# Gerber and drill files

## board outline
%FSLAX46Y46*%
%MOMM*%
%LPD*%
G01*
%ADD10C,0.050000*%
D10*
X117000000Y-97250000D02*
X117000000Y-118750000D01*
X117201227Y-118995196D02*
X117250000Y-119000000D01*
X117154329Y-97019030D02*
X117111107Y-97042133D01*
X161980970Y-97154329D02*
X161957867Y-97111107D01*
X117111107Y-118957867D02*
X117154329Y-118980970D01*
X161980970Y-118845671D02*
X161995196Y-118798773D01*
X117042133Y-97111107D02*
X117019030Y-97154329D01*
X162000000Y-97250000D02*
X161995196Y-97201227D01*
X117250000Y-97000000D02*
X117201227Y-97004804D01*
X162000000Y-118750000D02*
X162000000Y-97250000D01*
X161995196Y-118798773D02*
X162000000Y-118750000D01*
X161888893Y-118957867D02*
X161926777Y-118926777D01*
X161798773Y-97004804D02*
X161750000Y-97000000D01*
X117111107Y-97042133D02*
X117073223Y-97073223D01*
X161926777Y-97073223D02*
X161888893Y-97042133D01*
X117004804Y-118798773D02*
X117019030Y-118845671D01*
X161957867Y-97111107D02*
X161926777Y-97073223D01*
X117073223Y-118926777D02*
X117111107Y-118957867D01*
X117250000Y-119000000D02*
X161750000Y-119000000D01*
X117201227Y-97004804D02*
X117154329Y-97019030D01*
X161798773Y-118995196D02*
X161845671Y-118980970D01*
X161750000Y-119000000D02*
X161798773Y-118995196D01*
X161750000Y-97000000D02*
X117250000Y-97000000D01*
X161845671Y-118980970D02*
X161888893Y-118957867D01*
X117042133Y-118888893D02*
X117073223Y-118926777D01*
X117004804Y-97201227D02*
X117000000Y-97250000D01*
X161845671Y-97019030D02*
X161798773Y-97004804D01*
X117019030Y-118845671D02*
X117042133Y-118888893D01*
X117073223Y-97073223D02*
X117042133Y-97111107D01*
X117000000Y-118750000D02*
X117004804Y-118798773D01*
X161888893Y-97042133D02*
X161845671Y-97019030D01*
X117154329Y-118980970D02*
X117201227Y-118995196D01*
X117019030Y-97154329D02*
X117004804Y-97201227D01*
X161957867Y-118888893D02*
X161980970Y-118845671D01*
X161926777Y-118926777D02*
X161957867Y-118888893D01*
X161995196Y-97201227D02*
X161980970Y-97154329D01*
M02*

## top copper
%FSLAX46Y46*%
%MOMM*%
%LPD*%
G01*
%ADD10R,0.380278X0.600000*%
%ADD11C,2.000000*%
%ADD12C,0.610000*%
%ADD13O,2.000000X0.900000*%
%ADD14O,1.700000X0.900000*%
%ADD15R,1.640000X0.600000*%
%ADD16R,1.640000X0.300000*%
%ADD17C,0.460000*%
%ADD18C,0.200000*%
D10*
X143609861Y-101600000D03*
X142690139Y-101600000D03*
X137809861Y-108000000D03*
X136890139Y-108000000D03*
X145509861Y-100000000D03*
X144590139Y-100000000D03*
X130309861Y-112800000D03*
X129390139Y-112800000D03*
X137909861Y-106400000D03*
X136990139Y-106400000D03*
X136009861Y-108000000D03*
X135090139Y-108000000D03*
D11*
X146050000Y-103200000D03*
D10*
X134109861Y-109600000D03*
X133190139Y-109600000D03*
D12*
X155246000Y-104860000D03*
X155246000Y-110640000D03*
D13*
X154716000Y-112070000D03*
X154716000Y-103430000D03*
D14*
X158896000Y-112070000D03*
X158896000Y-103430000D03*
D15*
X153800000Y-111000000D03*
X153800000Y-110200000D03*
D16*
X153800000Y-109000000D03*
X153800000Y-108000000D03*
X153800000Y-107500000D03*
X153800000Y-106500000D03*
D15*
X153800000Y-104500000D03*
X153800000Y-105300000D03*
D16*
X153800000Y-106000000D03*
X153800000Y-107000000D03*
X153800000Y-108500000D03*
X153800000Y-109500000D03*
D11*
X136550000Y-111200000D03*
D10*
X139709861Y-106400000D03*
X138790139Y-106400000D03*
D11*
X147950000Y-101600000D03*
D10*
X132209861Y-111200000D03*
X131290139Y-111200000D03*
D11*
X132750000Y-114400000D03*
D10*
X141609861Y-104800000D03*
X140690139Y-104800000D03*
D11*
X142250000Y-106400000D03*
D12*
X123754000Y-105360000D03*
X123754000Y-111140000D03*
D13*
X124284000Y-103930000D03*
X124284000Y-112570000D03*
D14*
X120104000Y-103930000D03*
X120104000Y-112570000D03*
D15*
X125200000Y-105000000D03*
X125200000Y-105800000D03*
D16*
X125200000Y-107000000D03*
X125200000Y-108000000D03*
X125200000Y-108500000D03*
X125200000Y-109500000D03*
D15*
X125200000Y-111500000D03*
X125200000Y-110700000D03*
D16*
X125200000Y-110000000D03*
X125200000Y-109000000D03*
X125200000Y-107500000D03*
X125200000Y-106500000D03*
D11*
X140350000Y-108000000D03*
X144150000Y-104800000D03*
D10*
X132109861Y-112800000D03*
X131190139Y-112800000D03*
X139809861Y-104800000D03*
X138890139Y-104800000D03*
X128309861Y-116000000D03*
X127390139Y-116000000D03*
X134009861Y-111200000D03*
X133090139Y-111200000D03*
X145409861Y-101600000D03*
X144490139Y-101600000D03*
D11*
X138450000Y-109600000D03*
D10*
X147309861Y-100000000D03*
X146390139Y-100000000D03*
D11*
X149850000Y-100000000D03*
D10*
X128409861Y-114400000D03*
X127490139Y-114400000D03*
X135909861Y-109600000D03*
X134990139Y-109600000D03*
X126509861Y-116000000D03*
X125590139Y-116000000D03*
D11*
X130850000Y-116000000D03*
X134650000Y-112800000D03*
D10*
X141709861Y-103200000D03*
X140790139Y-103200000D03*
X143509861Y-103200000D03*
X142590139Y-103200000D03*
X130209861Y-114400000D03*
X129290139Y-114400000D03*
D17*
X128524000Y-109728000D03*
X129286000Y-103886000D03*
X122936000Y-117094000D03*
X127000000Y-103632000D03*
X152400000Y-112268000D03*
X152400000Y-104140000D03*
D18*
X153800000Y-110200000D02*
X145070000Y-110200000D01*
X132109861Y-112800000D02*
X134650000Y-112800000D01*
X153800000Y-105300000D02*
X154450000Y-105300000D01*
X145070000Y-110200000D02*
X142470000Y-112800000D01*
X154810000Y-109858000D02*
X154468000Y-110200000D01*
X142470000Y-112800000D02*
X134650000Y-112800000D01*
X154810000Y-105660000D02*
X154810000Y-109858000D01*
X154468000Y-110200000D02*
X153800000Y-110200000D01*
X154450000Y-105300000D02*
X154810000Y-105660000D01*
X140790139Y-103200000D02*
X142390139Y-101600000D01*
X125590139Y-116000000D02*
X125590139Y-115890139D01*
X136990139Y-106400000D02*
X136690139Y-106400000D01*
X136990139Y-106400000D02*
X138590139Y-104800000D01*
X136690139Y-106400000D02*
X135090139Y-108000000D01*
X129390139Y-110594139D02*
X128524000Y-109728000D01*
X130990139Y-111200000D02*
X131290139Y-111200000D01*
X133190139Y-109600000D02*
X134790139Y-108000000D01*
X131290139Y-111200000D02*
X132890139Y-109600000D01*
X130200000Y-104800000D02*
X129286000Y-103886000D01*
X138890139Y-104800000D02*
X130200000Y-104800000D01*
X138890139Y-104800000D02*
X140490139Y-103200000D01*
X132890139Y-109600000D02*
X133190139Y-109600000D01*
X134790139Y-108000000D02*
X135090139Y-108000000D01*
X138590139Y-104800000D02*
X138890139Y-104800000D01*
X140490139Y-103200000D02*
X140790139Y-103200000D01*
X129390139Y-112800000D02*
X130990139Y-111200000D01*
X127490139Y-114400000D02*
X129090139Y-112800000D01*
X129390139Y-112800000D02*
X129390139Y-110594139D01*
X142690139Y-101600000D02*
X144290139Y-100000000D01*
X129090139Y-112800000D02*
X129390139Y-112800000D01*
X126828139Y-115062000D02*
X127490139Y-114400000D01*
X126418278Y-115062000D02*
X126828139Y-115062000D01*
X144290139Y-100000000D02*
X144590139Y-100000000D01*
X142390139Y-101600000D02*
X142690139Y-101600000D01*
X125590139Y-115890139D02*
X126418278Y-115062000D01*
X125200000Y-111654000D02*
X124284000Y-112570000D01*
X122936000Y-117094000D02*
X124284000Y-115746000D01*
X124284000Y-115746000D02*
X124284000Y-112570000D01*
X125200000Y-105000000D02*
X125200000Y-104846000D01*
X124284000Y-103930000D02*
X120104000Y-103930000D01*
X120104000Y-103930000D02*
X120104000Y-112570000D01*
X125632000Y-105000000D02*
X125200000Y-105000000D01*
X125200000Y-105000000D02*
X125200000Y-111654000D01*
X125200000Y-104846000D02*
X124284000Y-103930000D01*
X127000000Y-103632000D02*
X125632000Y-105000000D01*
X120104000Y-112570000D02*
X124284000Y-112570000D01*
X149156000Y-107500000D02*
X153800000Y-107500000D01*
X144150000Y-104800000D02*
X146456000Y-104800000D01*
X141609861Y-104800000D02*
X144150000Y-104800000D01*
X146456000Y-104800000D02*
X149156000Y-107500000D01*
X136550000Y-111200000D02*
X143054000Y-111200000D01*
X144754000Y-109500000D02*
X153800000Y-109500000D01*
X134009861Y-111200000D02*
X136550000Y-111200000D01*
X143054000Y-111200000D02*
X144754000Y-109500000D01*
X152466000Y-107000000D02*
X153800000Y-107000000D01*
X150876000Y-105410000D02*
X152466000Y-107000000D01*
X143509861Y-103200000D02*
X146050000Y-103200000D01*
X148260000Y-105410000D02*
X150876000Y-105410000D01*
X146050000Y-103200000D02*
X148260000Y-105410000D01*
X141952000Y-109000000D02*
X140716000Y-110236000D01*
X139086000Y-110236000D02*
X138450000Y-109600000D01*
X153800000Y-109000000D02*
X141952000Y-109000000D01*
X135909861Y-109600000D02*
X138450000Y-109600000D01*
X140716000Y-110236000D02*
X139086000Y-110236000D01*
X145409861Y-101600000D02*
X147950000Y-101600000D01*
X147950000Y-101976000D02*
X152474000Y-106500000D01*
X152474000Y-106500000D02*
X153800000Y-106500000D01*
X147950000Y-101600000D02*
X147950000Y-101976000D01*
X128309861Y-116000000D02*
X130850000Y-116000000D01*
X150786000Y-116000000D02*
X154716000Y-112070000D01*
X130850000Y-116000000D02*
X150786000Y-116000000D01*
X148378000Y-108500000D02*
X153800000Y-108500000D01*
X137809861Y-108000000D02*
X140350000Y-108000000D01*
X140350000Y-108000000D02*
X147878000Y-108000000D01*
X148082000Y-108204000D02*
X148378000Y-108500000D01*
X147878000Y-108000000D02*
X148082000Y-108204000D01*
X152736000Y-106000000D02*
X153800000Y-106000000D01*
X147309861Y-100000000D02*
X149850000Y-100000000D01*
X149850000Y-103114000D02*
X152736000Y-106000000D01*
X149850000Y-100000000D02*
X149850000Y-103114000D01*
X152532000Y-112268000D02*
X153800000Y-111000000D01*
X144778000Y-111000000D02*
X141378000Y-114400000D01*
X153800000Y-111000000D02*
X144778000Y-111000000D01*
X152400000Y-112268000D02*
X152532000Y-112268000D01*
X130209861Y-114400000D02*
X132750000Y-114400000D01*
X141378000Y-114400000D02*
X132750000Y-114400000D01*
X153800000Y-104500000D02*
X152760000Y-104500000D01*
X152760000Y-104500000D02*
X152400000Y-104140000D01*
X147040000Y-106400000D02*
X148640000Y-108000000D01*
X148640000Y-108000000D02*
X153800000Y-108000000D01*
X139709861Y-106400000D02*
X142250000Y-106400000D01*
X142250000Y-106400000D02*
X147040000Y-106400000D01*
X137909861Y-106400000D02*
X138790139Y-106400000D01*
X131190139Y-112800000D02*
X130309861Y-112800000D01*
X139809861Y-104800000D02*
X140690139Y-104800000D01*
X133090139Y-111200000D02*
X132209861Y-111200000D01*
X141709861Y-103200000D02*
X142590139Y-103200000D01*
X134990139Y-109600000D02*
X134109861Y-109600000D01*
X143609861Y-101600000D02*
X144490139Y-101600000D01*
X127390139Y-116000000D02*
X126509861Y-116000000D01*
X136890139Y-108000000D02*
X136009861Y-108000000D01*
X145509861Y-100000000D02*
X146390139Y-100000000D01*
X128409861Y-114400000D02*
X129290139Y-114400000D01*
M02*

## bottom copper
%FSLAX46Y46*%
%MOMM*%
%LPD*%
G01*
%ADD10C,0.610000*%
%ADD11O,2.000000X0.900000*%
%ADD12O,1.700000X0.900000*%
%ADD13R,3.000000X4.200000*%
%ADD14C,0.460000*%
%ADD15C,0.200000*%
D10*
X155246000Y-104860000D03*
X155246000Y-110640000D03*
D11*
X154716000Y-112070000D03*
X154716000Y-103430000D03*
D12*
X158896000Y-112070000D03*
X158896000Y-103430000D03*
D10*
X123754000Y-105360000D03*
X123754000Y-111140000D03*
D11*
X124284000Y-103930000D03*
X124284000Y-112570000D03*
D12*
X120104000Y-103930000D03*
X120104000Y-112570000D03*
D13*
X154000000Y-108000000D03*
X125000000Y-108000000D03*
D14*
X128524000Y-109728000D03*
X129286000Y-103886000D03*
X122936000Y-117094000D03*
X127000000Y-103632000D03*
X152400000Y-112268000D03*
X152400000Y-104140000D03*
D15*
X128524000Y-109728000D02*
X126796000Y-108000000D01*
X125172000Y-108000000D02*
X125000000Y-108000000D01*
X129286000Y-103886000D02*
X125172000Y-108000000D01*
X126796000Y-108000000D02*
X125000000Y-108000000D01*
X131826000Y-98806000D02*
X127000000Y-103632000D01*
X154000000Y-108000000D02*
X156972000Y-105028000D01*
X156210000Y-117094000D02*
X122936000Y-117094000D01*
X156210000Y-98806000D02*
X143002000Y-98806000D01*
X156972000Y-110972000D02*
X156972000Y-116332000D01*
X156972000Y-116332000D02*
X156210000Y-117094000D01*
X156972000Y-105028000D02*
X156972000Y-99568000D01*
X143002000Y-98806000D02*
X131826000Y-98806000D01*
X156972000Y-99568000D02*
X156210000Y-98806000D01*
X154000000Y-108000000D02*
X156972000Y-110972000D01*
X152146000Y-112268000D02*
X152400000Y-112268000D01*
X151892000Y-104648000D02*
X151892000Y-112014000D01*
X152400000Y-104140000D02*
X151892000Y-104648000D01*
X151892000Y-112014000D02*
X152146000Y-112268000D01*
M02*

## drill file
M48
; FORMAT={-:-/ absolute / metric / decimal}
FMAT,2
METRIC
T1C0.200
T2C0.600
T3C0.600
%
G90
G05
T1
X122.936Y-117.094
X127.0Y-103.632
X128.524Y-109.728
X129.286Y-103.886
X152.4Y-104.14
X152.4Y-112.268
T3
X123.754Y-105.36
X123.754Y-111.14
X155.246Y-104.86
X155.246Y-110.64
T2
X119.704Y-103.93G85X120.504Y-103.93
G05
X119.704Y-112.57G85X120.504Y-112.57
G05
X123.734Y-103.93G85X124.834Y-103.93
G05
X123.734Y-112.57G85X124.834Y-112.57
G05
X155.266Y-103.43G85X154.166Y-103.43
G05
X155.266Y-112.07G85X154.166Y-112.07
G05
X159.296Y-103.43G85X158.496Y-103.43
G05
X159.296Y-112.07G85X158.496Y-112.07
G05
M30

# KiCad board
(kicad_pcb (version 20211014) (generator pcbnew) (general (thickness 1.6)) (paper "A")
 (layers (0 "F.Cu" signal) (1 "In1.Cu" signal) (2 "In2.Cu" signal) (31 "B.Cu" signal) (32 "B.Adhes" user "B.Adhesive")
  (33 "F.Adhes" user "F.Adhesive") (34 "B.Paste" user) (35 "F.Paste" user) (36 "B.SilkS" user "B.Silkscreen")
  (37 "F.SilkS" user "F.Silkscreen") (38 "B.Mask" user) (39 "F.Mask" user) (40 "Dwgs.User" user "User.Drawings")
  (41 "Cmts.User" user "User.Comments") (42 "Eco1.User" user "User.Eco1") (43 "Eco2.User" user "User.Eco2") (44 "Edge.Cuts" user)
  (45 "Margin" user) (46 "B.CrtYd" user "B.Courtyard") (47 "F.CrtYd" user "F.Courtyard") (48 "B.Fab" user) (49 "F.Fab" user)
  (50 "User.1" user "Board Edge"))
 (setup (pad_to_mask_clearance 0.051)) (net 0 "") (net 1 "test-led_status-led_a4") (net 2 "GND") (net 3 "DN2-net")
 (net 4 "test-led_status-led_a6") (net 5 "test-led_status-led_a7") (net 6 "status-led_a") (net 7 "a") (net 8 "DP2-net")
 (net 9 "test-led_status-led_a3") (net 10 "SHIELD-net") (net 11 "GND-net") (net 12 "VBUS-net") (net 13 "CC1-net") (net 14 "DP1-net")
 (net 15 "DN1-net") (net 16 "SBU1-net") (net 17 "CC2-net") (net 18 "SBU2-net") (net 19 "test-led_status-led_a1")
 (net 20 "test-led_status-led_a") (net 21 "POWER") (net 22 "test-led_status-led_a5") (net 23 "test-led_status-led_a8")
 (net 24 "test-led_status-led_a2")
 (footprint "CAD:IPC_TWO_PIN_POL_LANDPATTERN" (layer "F.Cu") (at 143.15 101.6 90)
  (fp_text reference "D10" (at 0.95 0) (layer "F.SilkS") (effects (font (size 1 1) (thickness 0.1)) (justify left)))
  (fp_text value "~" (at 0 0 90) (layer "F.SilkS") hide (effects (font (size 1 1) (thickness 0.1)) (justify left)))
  (pad "a" smd rect (at 0 0.459861 90) (size 0.6 0.380278) (layers "F.Cu" "F.Paste") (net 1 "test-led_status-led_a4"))
  (pad "c" smd rect (at 0 -0.459861 90) (size 0.6 0.380278) (layers "F.Cu" "F.Paste") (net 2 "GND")))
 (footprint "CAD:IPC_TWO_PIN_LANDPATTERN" (layer "F.Cu") (at 137.35 108 -90)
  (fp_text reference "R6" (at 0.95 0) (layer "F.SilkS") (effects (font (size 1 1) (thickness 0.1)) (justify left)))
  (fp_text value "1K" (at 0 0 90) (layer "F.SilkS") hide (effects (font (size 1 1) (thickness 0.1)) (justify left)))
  (pad "1" smd rect (at 0 -0.459861 270) (size 0.6 0.380278) (layers "F.Cu" "F.Paste") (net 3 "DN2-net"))
  (pad "2" smd rect (at 0 0.459861 270) (size 0.6 0.380278) (layers "F.Cu" "F.Paste") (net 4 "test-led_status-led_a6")))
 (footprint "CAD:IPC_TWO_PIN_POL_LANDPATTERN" (layer "F.Cu") (at 145.05 100 90)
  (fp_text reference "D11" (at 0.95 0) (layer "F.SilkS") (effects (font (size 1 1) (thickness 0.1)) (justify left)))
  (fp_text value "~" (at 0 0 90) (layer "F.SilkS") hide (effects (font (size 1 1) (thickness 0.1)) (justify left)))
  (pad "a" smd rect (at 0 0.459861 90) (size 0.6 0.380278) (layers "F.Cu" "F.Paste") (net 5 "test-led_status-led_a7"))
  (pad "c" smd rect (at 0 -0.459861 90) (size 0.6 0.380278) (layers "F.Cu" "F.Paste") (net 2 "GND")))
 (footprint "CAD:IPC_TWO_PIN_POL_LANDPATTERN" (layer "F.Cu") (at 129.85 112.8 90)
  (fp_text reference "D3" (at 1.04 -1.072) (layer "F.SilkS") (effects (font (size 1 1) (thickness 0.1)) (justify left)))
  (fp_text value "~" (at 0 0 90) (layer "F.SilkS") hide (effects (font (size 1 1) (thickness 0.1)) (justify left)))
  (pad "a" smd rect (at 0 0.459861 90) (size 0.6 0.380278) (layers "F.Cu" "F.Paste") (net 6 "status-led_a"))
  (pad "c" smd rect (at 0 -0.459861 90) (size 0.6 0.380278) (layers "F.Cu" "F.Paste") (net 2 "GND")))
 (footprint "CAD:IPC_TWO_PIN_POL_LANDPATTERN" (layer "F.Cu") (at 137.45 106.4 90)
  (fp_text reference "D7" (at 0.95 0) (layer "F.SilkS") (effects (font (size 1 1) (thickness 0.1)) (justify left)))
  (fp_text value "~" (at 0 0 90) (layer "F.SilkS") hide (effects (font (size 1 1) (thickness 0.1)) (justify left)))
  (pad "a" smd rect (at 0 0.459861 90) (size 0.6 0.380278) (layers "F.Cu" "F.Paste") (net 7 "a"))
  (pad "c" smd rect (at 0 -0.459861 90) (size 0.6 0.380278) (layers "F.Cu" "F.Paste") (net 2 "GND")))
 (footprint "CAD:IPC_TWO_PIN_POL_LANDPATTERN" (layer "F.Cu") (at 135.55 108 90)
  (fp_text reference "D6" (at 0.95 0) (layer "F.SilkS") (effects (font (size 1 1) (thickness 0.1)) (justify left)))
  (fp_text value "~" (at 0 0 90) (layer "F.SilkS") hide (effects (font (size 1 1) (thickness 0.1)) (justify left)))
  (pad "a" smd rect (at 0 0.459861 90) (size 0.6 0.380278) (layers "F.Cu" "F.Paste") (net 4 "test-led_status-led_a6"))
  (pad "c" smd rect (at 0 -0.459861 90) (size 0.6 0.380278) (layers "F.Cu" "F.Paste") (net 2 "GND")))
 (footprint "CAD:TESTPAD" (layer "F.Cu") (at 146.05 103.2)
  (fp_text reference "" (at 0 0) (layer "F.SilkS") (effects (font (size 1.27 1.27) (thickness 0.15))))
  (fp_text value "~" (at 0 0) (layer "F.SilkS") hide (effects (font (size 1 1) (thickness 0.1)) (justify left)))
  (pad "tp" smd circle (at 0 0) (size 2 2) (layers "F.Cu") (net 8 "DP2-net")))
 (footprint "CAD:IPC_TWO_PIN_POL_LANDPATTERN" (layer "F.Cu") (at 133.65 109.6 90)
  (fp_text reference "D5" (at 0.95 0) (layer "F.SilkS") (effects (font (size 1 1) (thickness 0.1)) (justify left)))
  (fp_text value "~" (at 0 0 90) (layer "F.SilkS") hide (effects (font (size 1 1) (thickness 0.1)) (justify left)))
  (pad "a" smd rect (at 0 0.459861 90) (size 0.6 0.380278) (layers "F.Cu" "F.Paste") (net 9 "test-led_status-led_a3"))
  (pad "c" smd rect (at 0 -0.459861 90) (size 0.6 0.380278) (layers "F.Cu" "F.Paste") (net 2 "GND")))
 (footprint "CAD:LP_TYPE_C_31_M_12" (layer "F.Cu") (at 153.8 111 90)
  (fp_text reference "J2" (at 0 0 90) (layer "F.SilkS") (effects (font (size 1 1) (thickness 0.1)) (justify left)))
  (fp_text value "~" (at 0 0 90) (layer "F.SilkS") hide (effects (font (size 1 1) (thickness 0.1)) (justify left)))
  (pad "" np_thru_hole circle (at 6.14 1.446 180) (size 0.61 0.61) (drill 0.6) (layers F&B.Cu *.Mask))
  (pad "" np_thru_hole circle (at 0.36 1.446 180) (size 0.61 0.61) (drill 0.6) (layers F&B.Cu *.Mask))
  (pad "13" thru_hole oval (at -1.07 0.916 180) (size 2 0.9) (drill oval 1.7 0.6) (layers *.Cu) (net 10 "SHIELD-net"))
  (pad "14" thru_hole oval (at 7.57 0.916 180) (size 2 0.9) (drill oval 1.7 0.6) (layers *.Cu) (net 10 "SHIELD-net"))
  (pad "15" thru_hole oval (at -1.07 5.096 180) (size 1.7 0.9) (drill oval 1.4 0.6) (layers *.Cu) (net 10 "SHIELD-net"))
  (pad "16" thru_hole oval (at 7.57 5.096 180) (size 1.7 0.9) (drill oval 1.4 0.6) (layers *.Cu) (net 10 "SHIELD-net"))
  (pad "A1-B12" smd rect (at 0 0 90) (size 0.6 1.64) (layers "F.Cu" "F.Paste") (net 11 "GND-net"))
  (pad "A4-B9" smd rect (at 0.8 0 90) (size 0.6 1.64) (layers "F.Cu" "F.Paste") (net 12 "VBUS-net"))
  (pad "A5" smd rect (at 2 0 90) (size 0.3 1.64) (layers "F.Cu" "F.Paste") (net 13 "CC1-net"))
  (pad "A6" smd rect (at 3 0 90) (size 0.3 1.64) (layers "F.Cu" "F.Paste") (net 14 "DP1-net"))
  (pad "A7" smd rect (at 3.5 0 90) (size 0.3 1.64) (layers "F.Cu" "F.Paste") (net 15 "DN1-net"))
  (pad "A8" smd rect (at 4.5 0 90) (size 0.3 1.64) (layers "F.Cu" "F.Paste") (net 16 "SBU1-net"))
  (pad "B1-A12" smd rect (at 6.5 0 90) (size 0.6 1.64) (layers "F.Cu" "F.Paste") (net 11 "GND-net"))
  (pad "B4-A9" smd rect (at 5.7 0 90) (size 0.6 1.64) (layers "F.Cu" "F.Paste") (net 12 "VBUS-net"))
  (pad "B5" smd rect (at 5 0 90) (size 0.3 1.64) (layers "F.Cu" "F.Paste") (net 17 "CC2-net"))
  (pad "B6" smd rect (at 4 0 90) (size 0.3 1.64) (layers "F.Cu" "F.Paste") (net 8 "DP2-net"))
  (pad "B7" smd rect (at 2.5 0 90) (size 0.3 1.64) (layers "F.Cu" "F.Paste") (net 3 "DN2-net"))
  (pad "B8" smd rect (at 1.5 0 90) (size 0.3 1.64) (layers "F.Cu" "F.Paste") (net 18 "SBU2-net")))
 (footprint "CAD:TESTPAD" (layer "F.Cu") (at 136.55 111.2)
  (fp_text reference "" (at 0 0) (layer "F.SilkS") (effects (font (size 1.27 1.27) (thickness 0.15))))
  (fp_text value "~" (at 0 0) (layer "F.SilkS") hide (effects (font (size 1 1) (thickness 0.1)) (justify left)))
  (pad "tp" smd circle (at 0 0) (size 2 2) (layers "F.Cu") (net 18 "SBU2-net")))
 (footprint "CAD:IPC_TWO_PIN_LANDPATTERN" (layer "F.Cu") (at 139.25 106.4 -90)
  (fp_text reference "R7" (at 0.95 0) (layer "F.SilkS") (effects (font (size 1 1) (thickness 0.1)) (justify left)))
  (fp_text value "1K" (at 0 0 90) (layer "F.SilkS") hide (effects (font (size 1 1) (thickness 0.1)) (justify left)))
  (pad "1" smd rect (at 0 -0.459861 270) (size 0.6 0.380278) (layers "F.Cu" "F.Paste") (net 14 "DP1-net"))
  (pad "2" smd rect (at 0 0.459861 270) (size 0.6 0.380278) (layers "F.Cu" "F.Paste") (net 7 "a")))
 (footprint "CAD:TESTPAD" (layer "F.Cu") (at 147.95 101.6)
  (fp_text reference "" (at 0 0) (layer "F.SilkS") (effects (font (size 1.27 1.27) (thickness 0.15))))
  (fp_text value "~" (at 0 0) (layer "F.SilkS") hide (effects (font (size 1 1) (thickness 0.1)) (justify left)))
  (pad "tp" smd circle (at 0 0) (size 2 2) (layers "F.Cu") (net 16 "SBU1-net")))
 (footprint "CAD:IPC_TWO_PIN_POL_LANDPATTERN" (layer "F.Cu") (at 131.75 111.2 90)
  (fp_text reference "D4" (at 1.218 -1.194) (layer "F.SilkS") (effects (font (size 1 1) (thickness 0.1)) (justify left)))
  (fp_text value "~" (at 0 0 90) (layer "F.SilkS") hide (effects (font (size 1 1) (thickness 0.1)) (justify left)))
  (pad "a" smd rect (at 0 0.459861 90) (size 0.6 0.380278) (layers "F.Cu" "F.Paste") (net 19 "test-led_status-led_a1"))
  (pad "c" smd rect (at 0 -0.459861 90) (size 0.6 0.380278) (layers "F.Cu" "F.Paste") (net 2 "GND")))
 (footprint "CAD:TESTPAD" (layer "F.Cu") (at 132.75 114.4)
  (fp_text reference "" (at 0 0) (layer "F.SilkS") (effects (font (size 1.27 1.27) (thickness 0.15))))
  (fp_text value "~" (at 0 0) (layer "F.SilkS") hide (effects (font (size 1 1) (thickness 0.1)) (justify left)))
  (pad "tp" smd circle (at 0 0) (size 2 2) (layers "F.Cu") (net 11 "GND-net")))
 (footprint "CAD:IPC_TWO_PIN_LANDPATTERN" (layer "F.Cu") (at 141.15 104.8 -90)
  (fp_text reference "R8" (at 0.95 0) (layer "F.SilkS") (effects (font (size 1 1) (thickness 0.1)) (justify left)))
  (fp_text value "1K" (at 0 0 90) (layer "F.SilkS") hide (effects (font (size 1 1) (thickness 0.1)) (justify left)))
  (pad "1" smd rect (at 0 -0.459861 270) (size 0.6 0.380278) (layers "F.Cu" "F.Paste") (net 15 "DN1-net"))
  (pad "2" smd rect (at 0 0.459861 270) (size 0.6 0.380278) (layers "F.Cu" "F.Paste") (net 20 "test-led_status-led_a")))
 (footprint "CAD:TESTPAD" (layer "F.Cu") (at 142.25 106.4)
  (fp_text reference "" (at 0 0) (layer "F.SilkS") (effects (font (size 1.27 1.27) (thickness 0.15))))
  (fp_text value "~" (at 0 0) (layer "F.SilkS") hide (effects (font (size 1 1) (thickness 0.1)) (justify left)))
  (pad "tp" smd circle (at 0 0) (size 2 2) (layers "F.Cu") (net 14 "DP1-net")))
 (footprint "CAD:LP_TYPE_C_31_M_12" (layer "F.Cu") (at 125.2 105 -90)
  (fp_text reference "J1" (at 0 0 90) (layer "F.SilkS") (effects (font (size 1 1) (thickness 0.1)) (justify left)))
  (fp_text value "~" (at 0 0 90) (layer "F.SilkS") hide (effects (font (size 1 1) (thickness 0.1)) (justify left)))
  (pad "" np_thru_hole circle (at 0.36 1.446) (size 0.61 0.61) (drill 0.6) (layers F&B.Cu *.Mask))
  (pad "" np_thru_hole circle (at 6.14 1.446) (size 0.61 0.61) (drill 0.6) (layers F&B.Cu *.Mask))
  (pad "13" thru_hole oval (at -1.07 0.916) (size 2 0.9) (drill oval 1.7 0.6) (layers *.Cu) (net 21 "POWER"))
  (pad "14" thru_hole oval (at 7.57 0.916) (size 2 0.9) (drill oval 1.7 0.6) (layers *.Cu) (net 21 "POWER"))
  (pad "15" thru_hole oval (at -1.07 5.096) (size 1.7 0.9) (drill oval 1.4 0.6) (layers *.Cu) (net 21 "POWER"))
  (pad "16" thru_hole oval (at 7.57 5.096) (size 1.7 0.9) (drill oval 1.4 0.6) (layers *.Cu) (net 21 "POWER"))
  (pad "A1-B12" smd rect (at 0 0 270) (size 0.6 1.64) (layers "F.Cu" "F.Paste") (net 21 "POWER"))
  (pad "A4-B9" smd rect (at 0.8 0 270) (size 0.6 1.64) (layers "F.Cu" "F.Paste") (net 21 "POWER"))
  (pad "A5" smd rect (at 2 0 270) (size 0.3 1.64) (layers "F.Cu" "F.Paste") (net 21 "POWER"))
  (pad "A6" smd rect (at 3 0 270) (size 0.3 1.64) (layers "F.Cu" "F.Paste") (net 21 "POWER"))
  (pad "A7" smd rect (at 3.5 0 270) (size 0.3 1.64) (layers "F.Cu" "F.Paste") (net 21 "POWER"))
  (pad "A8" smd rect (at 4.5 0 270) (size 0.3 1.64) (layers "F.Cu" "F.Paste") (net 21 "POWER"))
  (pad "B1-A12" smd rect (at 6.5 0 270) (size 0.6 1.64) (layers "F.Cu" "F.Paste") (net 21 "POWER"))
  (pad "B4-A9" smd rect (at 5.7 0 270) (size 0.6 1.64) (layers "F.Cu" "F.Paste") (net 21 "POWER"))
  (pad "B5" smd rect (at 5 0 270) (size 0.3 1.64) (layers "F.Cu" "F.Paste") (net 21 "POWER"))
  (pad "B6" smd rect (at 4 0 270) (size 0.3 1.64) (layers "F.Cu" "F.Paste") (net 21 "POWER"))
  (pad "B7" smd rect (at 2.5 0 270) (size 0.3 1.64) (layers "F.Cu" "F.Paste") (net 21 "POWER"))
  (pad "B8" smd rect (at 1.5 0 270) (size 0.3 1.64) (layers "F.Cu" "F.Paste") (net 21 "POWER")))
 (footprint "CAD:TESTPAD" (layer "F.Cu") (at 140.35 108)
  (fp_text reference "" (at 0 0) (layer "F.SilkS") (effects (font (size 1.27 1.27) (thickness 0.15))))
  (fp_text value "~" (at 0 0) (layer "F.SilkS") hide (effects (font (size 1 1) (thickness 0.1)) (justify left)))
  (pad "tp" smd circle (at 0 0) (size 2 2) (layers "F.Cu") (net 3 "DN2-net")))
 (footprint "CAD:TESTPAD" (layer "F.Cu") (at 144.15 104.8)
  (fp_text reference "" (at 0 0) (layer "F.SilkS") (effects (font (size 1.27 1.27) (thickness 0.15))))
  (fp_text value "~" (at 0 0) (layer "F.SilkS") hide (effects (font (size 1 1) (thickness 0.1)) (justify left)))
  (pad "tp" smd circle (at 0 0) (size 2 2) (layers "F.Cu") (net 15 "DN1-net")))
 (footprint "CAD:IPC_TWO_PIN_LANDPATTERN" (layer "F.Cu") (at 131.65 112.8 -90)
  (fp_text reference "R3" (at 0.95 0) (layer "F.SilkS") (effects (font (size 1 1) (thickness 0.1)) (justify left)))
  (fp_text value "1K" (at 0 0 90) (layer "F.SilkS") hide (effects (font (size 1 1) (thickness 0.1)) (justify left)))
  (pad "1" smd rect (at 0 -0.459861 270) (size 0.6 0.380278) (layers "F.Cu" "F.Paste") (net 12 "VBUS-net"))
  (pad "2" smd rect (at 0 0.459861 270) (size 0.6 0.380278) (layers "F.Cu" "F.Paste") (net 6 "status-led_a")))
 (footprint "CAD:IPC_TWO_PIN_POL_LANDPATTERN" (layer "F.Cu") (at 139.35 104.8 90)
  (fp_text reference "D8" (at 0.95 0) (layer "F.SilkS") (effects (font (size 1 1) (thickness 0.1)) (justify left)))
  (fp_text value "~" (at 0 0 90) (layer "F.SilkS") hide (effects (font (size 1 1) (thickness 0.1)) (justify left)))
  (pad "a" smd rect (at 0 0.459861 90) (size 0.6 0.380278) (layers "F.Cu" "F.Paste") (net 20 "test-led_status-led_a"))
  (pad "c" smd rect (at 0 -0.459861 90) (size 0.6 0.380278) (layers "F.Cu" "F.Paste") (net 2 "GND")))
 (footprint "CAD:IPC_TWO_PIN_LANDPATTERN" (layer "F.Cu") (at 127.85 116 -90)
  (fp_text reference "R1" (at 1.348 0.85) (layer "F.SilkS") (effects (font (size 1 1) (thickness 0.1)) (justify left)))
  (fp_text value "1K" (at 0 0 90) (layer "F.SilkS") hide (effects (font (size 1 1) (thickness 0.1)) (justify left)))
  (pad "1" smd rect (at 0 -0.459861 270) (size 0.6 0.380278) (layers "F.Cu" "F.Paste") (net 10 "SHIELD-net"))
  (pad "2" smd rect (at 0 0.459861 270) (size 0.6 0.380278) (layers "F.Cu" "F.Paste") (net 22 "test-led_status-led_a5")))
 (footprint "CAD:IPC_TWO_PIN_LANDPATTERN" (layer "F.Cu") (at 133.55 111.2 -90)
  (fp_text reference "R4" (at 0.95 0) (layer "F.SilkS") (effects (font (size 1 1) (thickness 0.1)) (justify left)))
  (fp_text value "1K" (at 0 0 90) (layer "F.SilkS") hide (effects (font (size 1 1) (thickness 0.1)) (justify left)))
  (pad "1" smd rect (at 0 -0.459861 270) (size 0.6 0.380278) (layers "F.Cu" "F.Paste") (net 18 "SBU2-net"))
  (pad "2" smd rect (at 0 0.459861 270) (size 0.6 0.380278) (layers "F.Cu" "F.Paste") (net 19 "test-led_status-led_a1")))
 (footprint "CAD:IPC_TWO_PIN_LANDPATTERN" (layer "F.Cu") (at 144.95 101.6 -90)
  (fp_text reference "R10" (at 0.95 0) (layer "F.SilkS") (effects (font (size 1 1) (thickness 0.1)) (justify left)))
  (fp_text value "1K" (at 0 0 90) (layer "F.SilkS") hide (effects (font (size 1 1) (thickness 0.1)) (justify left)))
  (pad "1" smd rect (at 0 -0.459861 270) (size 0.6 0.380278) (layers "F.Cu" "F.Paste") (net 16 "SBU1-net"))
  (pad "2" smd rect (at 0 0.459861 270) (size 0.6 0.380278) (layers "F.Cu" "F.Paste") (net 1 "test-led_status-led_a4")))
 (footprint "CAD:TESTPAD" (layer "F.Cu") (at 138.45 109.6)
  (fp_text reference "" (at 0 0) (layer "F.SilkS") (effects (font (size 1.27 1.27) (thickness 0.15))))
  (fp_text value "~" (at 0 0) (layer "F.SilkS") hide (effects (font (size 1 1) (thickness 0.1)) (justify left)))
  (pad "tp" smd circle (at 0 0) (size 2 2) (layers "F.Cu") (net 13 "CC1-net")))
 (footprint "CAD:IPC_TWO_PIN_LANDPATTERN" (layer "F.Cu") (at 146.85 100 -90)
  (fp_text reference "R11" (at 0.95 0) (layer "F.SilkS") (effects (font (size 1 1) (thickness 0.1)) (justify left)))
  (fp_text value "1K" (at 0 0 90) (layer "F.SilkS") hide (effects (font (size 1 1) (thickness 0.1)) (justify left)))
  (pad "1" smd rect (at 0 -0.459861 270) (size 0.6 0.380278) (layers "F.Cu" "F.Paste") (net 17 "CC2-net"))
  (pad "2" smd rect (at 0 0.459861 270) (size 0.6 0.380278) (layers "F.Cu" "F.Paste") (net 5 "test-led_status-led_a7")))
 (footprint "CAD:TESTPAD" (layer "F.Cu") (at 149.85 100)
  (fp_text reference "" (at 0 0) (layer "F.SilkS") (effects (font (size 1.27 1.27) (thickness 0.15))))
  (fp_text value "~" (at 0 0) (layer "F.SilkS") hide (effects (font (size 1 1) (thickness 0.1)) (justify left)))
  (pad "tp" smd circle (at 0 0) (size 2 2) (layers "F.Cu") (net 17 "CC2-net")))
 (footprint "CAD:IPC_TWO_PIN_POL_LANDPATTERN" (layer "F.Cu") (at 127.95 114.4 90)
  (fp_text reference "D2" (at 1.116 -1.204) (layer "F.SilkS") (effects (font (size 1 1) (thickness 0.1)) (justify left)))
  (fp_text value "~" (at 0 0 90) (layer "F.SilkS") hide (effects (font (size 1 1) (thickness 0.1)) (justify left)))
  (pad "a" smd rect (at 0 0.459861 90) (size 0.6 0.380278) (layers "F.Cu" "F.Paste") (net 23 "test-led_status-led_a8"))
  (pad "c" smd rect (at 0 -0.459861 90) (size 0.6 0.380278) (layers "F.Cu" "F.Paste") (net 2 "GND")))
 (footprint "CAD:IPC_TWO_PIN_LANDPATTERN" (layer "F.Cu") (at 135.45 109.6 -90)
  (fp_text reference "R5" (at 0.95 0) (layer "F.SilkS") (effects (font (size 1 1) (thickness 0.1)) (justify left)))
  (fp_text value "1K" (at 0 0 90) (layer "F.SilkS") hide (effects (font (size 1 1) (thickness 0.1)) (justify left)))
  (pad "1" smd rect (at 0 -0.459861 270) (size 0.6 0.380278) (layers "F.Cu" "F.Paste") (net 13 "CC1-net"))
  (pad "2" smd rect (at 0 0.459861 270) (size 0.6 0.380278) (layers "F.Cu" "F.Paste") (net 9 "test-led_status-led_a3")))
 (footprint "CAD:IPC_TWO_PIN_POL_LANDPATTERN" (layer "F.Cu") (at 126.05 116 90)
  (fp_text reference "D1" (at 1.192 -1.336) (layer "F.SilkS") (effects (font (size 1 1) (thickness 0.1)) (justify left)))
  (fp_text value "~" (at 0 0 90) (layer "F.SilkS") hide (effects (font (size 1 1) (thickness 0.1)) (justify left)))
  (pad "a" smd rect (at 0 0.459861 90) (size 0.6 0.380278) (layers "F.Cu" "F.Paste") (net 22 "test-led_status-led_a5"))
  (pad "c" smd rect (at 0 -0.459861 90) (size 0.6 0.380278) (layers "F.Cu" "F.Paste") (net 2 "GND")))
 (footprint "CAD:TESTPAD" (layer "F.Cu") (at 130.85 116)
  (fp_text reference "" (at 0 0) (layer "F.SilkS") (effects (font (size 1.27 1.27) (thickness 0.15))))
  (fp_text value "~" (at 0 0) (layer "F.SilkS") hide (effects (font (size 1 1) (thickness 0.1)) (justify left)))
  (pad "tp" smd circle (at 0 0) (size 2 2) (layers "F.Cu") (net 10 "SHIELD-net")))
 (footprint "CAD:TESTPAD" (layer "F.Cu") (at 134.65 112.8)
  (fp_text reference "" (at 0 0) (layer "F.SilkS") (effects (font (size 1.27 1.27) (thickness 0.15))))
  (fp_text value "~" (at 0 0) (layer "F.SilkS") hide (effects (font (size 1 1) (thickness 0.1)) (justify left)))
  (pad "tp" smd circle (at 0 0) (size 2 2) (layers "F.Cu") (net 12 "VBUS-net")))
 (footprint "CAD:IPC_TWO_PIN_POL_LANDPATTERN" (layer "F.Cu") (at 141.25 103.2 90)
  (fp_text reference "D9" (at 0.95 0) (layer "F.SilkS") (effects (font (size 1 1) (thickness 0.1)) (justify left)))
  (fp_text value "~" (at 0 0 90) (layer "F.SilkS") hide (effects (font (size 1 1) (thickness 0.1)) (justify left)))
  (pad "a" smd rect (at 0 0.459861 90) (size 0.6 0.380278) (layers "F.Cu" "F.Paste") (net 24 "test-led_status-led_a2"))
  (pad "c" smd rect (at 0 -0.459861 90) (size 0.6 0.380278) (layers "F.Cu" "F.Paste") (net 2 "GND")))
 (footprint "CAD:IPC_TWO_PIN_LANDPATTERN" (layer "F.Cu") (at 143.05 103.2 -90)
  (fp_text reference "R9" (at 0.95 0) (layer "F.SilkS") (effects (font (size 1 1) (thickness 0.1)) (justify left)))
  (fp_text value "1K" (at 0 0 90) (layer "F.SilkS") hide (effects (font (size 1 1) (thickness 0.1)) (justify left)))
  (pad "1" smd rect (at 0 -0.459861 270) (size 0.6 0.380278) (layers "F.Cu" "F.Paste") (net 8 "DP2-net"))
  (pad "2" smd rect (at 0 0.459861 270) (size 0.6 0.380278) (layers "F.Cu" "F.Paste") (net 24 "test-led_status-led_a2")))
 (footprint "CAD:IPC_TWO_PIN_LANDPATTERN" (layer "F.Cu") (at 129.75 114.4 -90)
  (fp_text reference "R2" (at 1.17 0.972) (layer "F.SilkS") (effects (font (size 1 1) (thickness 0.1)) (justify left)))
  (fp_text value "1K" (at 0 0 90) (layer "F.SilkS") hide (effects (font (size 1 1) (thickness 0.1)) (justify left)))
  (pad "1" smd rect (at 0 -0.459861 270) (size 0.6 0.380278) (layers "F.Cu" "F.Paste") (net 11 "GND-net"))
  (pad "2" smd rect (at 0 0.459861 270) (size 0.6 0.380278) (layers "F.Cu" "F.Paste") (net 23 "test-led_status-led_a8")))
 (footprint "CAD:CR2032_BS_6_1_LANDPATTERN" (layer "B.Cu") (at 139.5 108 -90)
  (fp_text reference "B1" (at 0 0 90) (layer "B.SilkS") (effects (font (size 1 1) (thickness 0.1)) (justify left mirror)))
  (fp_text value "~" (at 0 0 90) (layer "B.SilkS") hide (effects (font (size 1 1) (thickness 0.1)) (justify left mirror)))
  (pad "1" smd rect (at 0 -14.5 270) (size 4.2 3) (layers "B.Cu" "B.Paste") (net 21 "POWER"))
  (pad "2" smd rect (at 0 14.5 270) (size 4.2 3) (layers "B.Cu" "B.Paste") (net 2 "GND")))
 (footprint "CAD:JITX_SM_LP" (layer "B.Cu") (at 149.5 113)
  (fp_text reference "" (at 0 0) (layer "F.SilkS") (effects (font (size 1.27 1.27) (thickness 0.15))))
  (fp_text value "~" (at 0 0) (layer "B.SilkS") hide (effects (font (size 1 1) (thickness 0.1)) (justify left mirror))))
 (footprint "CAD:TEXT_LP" (layer "B.Cu") (at 154.94 98.298)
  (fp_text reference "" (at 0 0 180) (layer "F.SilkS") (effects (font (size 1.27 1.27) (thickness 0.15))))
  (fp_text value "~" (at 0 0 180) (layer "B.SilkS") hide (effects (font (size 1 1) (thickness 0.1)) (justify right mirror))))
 (gr_line (start 117 97.25) (end 117 118.75) (layer "Edge.Cuts") (width 0.05))
 (gr_line (start 117.201227 118.995196) (end 117.25 119) (layer "Edge.Cuts") (width 0.05))
 (gr_line (start 117.154329 97.01903) (end 117.111107 97.042133) (layer "Edge.Cuts") (width 0.05))
 (gr_line (start 161.98097 97.154329) (end 161.957867 97.111107) (layer "Edge.Cuts") (width 0.05))
 (gr_line (start 117.111107 118.957867) (end 117.154329 118.98097) (layer "Edge.Cuts") (width 0.05))
 (gr_line (start 161.98097 118.845671) (end 161.995196 118.798773) (layer "Edge.Cuts") (width 0.05))
 (gr_line (start 117.042133 97.111107) (end 117.01903 97.154329) (layer "Edge.Cuts") (width 0.05))
 (gr_line (start 162 97.25) (end 161.995196 97.201227) (layer "Edge.Cuts") (width 0.05))
 (gr_line (start 117.25 97) (end 117.201227 97.004804) (layer "Edge.Cuts") (width 0.05))
 (gr_line (start 162 118.75) (end 162 97.25) (layer "Edge.Cuts") (width 0.05))
 (gr_line (start 161.995196 118.798773) (end 162 118.75) (layer "Edge.Cuts") (width 0.05))
 (gr_line (start 161.888893 118.957867) (end 161.926777 118.926777) (layer "Edge.Cuts") (width 0.05))
 (gr_line (start 161.798773 97.004804) (end 161.75 97) (layer "Edge.Cuts") (width 0.05))
 (gr_line (start 117.111107 97.042133) (end 117.073223 97.073223) (layer "Edge.Cuts") (width 0.05))
 (gr_line (start 161.926777 97.073223) (end 161.888893 97.042133) (layer "Edge.Cuts") (width 0.05))
 (gr_line (start 117.004804 118.798773) (end 117.01903 118.845671) (layer "Edge.Cuts") (width 0.05))
 (gr_line (start 161.957867 97.111107) (end 161.926777 97.073223) (layer "Edge.Cuts") (width 0.05))
 (gr_line (start 117.073223 118.926777) (end 117.111107 118.957867) (layer "Edge.Cuts") (width 0.05))
 (gr_line (start 117.25 119) (end 161.75 119) (layer "Edge.Cuts") (width 0.05))
 (gr_line (start 117.201227 97.004804) (end 117.154329 97.01903) (layer "Edge.Cuts") (width 0.05))
 (gr_line (start 161.798773 118.995196) (end 161.845671 118.98097) (layer "Edge.Cuts") (width 0.05))
 (gr_line (start 161.75 119) (end 161.798773 118.995196) (layer "Edge.Cuts") (width 0.05))
 (gr_line (start 161.75 97) (end 117.25 97) (layer "Edge.Cuts") (width 0.05))
 (gr_line (start 161.845671 118.98097) (end 161.888893 118.957867) (layer "Edge.Cuts") (width 0.05))
 (gr_line (start 117.042133 118.888893) (end 117.073223 118.926777) (layer "Edge.Cuts") (width 0.05))
 (gr_line (start 117.004804 97.201227) (end 117 97.25) (layer "Edge.Cuts") (width 0.05))
 (gr_line (start 161.845671 97.01903) (end 161.798773 97.004804) (layer "Edge.Cuts") (width 0.05))
 (gr_line (start 117.01903 118.845671) (end 117.042133 118.888893) (layer "Edge.Cuts") (width 0.05))
 (gr_line (start 117.073223 97.073223) (end 117.042133 97.111107) (layer "Edge.Cuts") (width 0.05))
 (gr_line (start 117 118.75) (end 117.004804 118.798773) (layer "Edge.Cuts") (width 0.05))
 (gr_line (start 161.888893 97.042133) (end 161.845671 97.01903) (layer "Edge.Cuts") (width 0.05))
 (gr_line (start 117.154329 118.98097) (end 117.201227 118.995196) (layer "Edge.Cuts") (width 0.05))
 (gr_line (start 117.01903 97.154329) (end 117.004804 97.201227) (layer "Edge.Cuts") (width 0.05))
 (gr_line (start 161.957867 118.888893) (end 161.98097 118.845671) (layer "Edge.Cuts") (width 0.05))
 (gr_line (start 161.926777 118.926777) (end 161.957867 118.888893) (layer "Edge.Cuts") (width 0.05))
 (gr_line (start 161.995196 97.201227) (end 161.98097 97.154329) (layer "Edge.Cuts") (width 0.05))
 (segment (start 153.8 110.2) (end 145.07 110.2) (width 0.2) (layer "F.Cu") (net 12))
 (segment (start 132.109861 112.8) (end 134.65 112.8) (width 0.2) (layer "F.Cu") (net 12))
 (segment (start 153.8 105.3) (end 154.45 105.3) (width 0.2) (layer "F.Cu") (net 12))
 (segment (start 145.07 110.2) (end 142.47 112.8) (width 0.2) (layer "F.Cu") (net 12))
 (segment (start 154.81 109.858) (end 154.468 110.2) (width 0.2) (layer "F.Cu") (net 12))
 (segment (start 142.47 112.8) (end 134.65 112.8) (width 0.2) (layer "F.Cu") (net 12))
 (segment (start 154.81 105.66) (end 154.81 109.858) (width 0.2) (layer "F.Cu") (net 12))
 (segment (start 154.468 110.2) (end 153.8 110.2) (width 0.2) (layer "F.Cu") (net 12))
 (segment (start 154.45 105.3) (end 154.81 105.66) (width 0.2) (layer "F.Cu") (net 12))
 (segment (start 140.790139 103.2) (end 142.390139 101.6) (width 0.2) (layer "F.Cu") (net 2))
 (segment (start 125.590139 116) (end 125.590139 115.890139) (width 0.2) (layer "F.Cu") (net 2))
 (segment (start 136.990139 106.4) (end 136.690139 106.4) (width 0.2) (layer "F.Cu") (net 2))
 (segment (start 136.990139 106.4) (end 138.590139 104.8) (width 0.2) (layer "F.Cu") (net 2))
 (segment (start 136.690139 106.4) (end 135.090139 108) (width 0.2) (layer "F.Cu") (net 2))
 (segment (start 129.390139 110.594139) (end 128.524 109.728) (width 0.2) (layer "F.Cu") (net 2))
 (segment (start 130.990139 111.2) (end 131.290139 111.2) (width 0.2) (layer "F.Cu") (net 2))
 (segment (start 133.190139 109.6) (end 134.790139 108) (width 0.2) (layer "F.Cu") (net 2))
 (segment (start 131.290139 111.2) (end 132.890139 109.6) (width 0.2) (layer "F.Cu") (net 2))
 (segment (start 130.2 104.8) (end 129.286 103.886) (width 0.2) (layer "F.Cu") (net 2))
 (segment (start 138.890139 104.8) (end 130.2 104.8) (width 0.2) (layer "F.Cu") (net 2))
 (segment (start 138.890139 104.8) (end 140.490139 103.2) (width 0.2) (layer "F.Cu") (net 2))
 (segment (start 132.890139 109.6) (end 133.190139 109.6) (width 0.2) (layer "F.Cu") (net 2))
 (segment (start 134.790139 108) (end 135.090139 108) (width 0.2) (layer "F.Cu") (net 2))
 (segment (start 138.590139 104.8) (end 138.890139 104.8) (width 0.2) (layer "F.Cu") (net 2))
 (segment (start 140.490139 103.2) (end 140.790139 103.2) (width 0.2) (layer "F.Cu") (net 2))
 (segment (start 129.390139 112.8) (end 130.990139 111.2) (width 0.2) (layer "F.Cu") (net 2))
 (segment (start 127.490139 114.4) (end 129.090139 112.8) (width 0.2) (layer "F.Cu") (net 2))
 (segment (start 129.390139 112.8) (end 129.390139 110.594139) (width 0.2) (layer "F.Cu") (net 2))
 (segment (start 142.690139 101.6) (end 144.290139 100) (width 0.2) (layer "F.Cu") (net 2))
 (segment (start 129.090139 112.8) (end 129.390139 112.8) (width 0.2) (layer "F.Cu") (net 2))
 (segment (start 126.828139 115.062) (end 127.490139 114.4) (width 0.2) (layer "F.Cu") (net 2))
 (segment (start 126.418278 115.062) (end 126.828139 115.062) (width 0.2) (layer "F.Cu") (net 2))
 (segment (start 144.290139 100) (end 144.590139 100) (width 0.2) (layer "F.Cu") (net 2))
 (segment (start 142.390139 101.6) (end 142.690139 101.6) (width 0.2) (layer "F.Cu") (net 2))
 (segment (start 125.590139 115.890139) (end 126.418278 115.062) (width 0.2) (layer "F.Cu") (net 2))
 (via (at 128.524 109.728) (size 0.46) (drill 0.2) (layers "F.Cu" "B.Cu") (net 2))
 (via (at 129.286 103.886) (size 0.46) (drill 0.2) (layers "F.Cu" "B.Cu") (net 2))
 (segment (start 128.524 109.728) (end 126.796 108) (width 0.2) (layer "B.Cu") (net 2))
 (segment (start 125.172 108) (end 125 108) (width 0.2) (layer "B.Cu") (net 2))
 (segment (start 129.286 103.886) (end 125.172 108) (width 0.2) (layer "B.Cu") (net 2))
 (segment (start 126.796 108) (end 125 108) (width 0.2) (layer "B.Cu") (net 2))
 (segment (start 125.2 111.654) (end 124.284 112.57) (width 0.2) (layer "F.Cu") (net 21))
 (segment (start 122.936 117.094) (end 124.284 115.746) (width 0.2) (layer "F.Cu") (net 21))
 (segment (start 124.284 115.746) (end 124.284 112.57) (width 0.2) (layer "F.Cu") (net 21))
 (segment (start 125.2 105) (end 125.2 104.846) (width 0.2) (layer "F.Cu") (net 21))
 (segment (start 124.284 103.93) (end 120.104 103.93) (width 0.2) (layer "F.Cu") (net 21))
 (segment (start 120.104 103.93) (end 120.104 112.57) (width 0.2) (layer "F.Cu") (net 21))
 (segment (start 125.632 105) (end 125.2 105) (width 0.2) (layer "F.Cu") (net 21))
 (segment (start 125.2 105) (end 125.2 111.654) (width 0.2) (layer "F.Cu") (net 21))
 (segment (start 125.2 104.846) (end 124.284 103.93) (width 0.2) (layer "F.Cu") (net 21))
 (segment (start 127 103.632) (end 125.632 105) (width 0.2) (layer "F.Cu") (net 21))
 (segment (start 120.104 112.57) (end 124.284 112.57) (width 0.2) (layer "F.Cu") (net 21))
 (via (at 122.936 117.094) (size 0.46) (drill 0.2) (layers "F.Cu" "B.Cu") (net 21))
 (via (at 127 103.632) (size 0.46) (drill 0.2) (layers "F.Cu" "B.Cu") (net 21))
 (segment (start 131.826 98.806) (end 127 103.632) (width 0.2) (layer "B.Cu") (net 21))
 (segment (start 154 108) (end 156.972 105.028) (width 0.2) (layer "B.Cu") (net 21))
 (segment (start 156.21 117.094) (end 122.936 117.094) (width 0.2) (layer "B.Cu") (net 21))
 (segment (start 156.21 98.806) (end 143.002 98.806) (width 0.2) (layer "B.Cu") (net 21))
 (segment (start 156.972 110.972) (end 156.972 116.332) (width 0.2) (layer "B.Cu") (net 21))
 (segment (start 156.972 116.332) (end 156.21 117.094) (width 0.2) (layer "B.Cu") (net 21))
 (segment (start 156.972 105.028) (end 156.972 99.568) (width 0.2) (layer "B.Cu") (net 21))
 (segment (start 143.002 98.806) (end 131.826 98.806) (width 0.2) (layer "B.Cu") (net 21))
 (segment (start 156.972 99.568) (end 156.21 98.806) (width 0.2) (layer "B.Cu") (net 21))
 (segment (start 154 108) (end 156.972 110.972) (width 0.2) (layer "B.Cu") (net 21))
 (segment (start 149.156 107.5) (end 153.8 107.5) (width 0.2) (layer "F.Cu") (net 15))
 (segment (start 144.15 104.8) (end 146.456 104.8) (width 0.2) (layer "F.Cu") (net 15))
 (segment (start 141.609861 104.8) (end 144.15 104.8) (width 0.2) (layer "F.Cu") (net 15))
 (segment (start 146.456 104.8) (end 149.156 107.5) (width 0.2) (layer "F.Cu") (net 15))
 (segment (start 136.55 111.2) (end 143.054 111.2) (width 0.2) (layer "F.Cu") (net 18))
 (segment (start 144.754 109.5) (end 153.8 109.5) (width 0.2) (layer "F.Cu") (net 18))
 (segment (start 134.009861 111.2) (end 136.55 111.2) (width 0.2) (layer "F.Cu") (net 18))
 (segment (start 143.054 111.2) (end 144.754 109.5) (width 0.2) (layer "F.Cu") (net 18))
 (segment (start 152.466 107) (end 153.8 107) (width 0.2) (layer "F.Cu") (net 8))
 (segment (start 150.876 105.41) (end 152.466 107) (width 0.2) (layer "F.Cu") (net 8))
 (segment (start 143.509861 103.2) (end 146.05 103.2) (width 0.2) (layer "F.Cu") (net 8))
 (segment (start 148.26 105.41) (end 150.876 105.41) (width 0.2) (layer "F.Cu") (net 8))
 (segment (start 146.05 103.2) (end 148.26 105.41) (width 0.2) (layer "F.Cu") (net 8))
 (segment (start 141.952 109) (end 140.716 110.236) (width 0.2) (layer "F.Cu") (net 13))
 (segment (start 139.086 110.236) (end 138.45 109.6) (width 0.2) (layer "F.Cu") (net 13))
 (segment (start 153.8 109) (end 141.952 109) (width 0.2) (layer "F.Cu") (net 13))
 (segment (start 135.909861 109.6) (end 138.45 109.6) (width 0.2) (layer "F.Cu") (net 13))
 (segment (start 140.716 110.236) (end 139.086 110.236) (width 0.2) (layer "F.Cu") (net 13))
 (segment (start 145.409861 101.6) (end 147.95 101.6) (width 0.2) (layer "F.Cu") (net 16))
 (segment (start 147.95 101.976) (end 152.474 106.5) (width 0.2) (layer "F.Cu") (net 16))
 (segment (start 152.474 106.5) (end 153.8 106.5) (width 0.2) (layer "F.Cu") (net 16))
 (segment (start 147.95 101.6) (end 147.95 101.976) (width 0.2) (layer "F.Cu") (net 16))
 (segment (start 128.309861 116) (end 130.85 116) (width 0.2) (layer "F.Cu") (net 10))
 (segment (start 150.786 116) (end 154.716 112.07) (width 0.2) (layer "F.Cu") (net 10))
 (segment (start 130.85 116) (end 150.786 116) (width 0.2) (layer "F.Cu") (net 10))
 (segment (start 148.378 108.5) (end 153.8 108.5) (width 0.2) (layer "F.Cu") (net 3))
 (segment (start 137.809861 108) (end 140.35 108) (width 0.2) (layer "F.Cu") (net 3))
 (segment (start 140.35 108) (end 147.878 108) (width 0.2) (layer "F.Cu") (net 3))
 (segment (start 148.082 108.204) (end 148.378 108.5) (width 0.2) (layer "F.Cu") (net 3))
 (segment (start 147.878 108) (end 148.082 108.204) (width 0.2) (layer "F.Cu") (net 3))
 (segment (start 152.736 106) (end 153.8 106) (width 0.2) (layer "F.Cu") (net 17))
 (segment (start 147.309861 100) (end 149.85 100) (width 0.2) (layer "F.Cu") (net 17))
 (segment (start 149.85 103.114) (end 152.736 106) (width 0.2) (layer "F.Cu") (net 17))
 (segment (start 149.85 100) (end 149.85 103.114) (width 0.2) (layer "F.Cu") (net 17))
 (segment (start 152.532 112.268) (end 153.8 111) (width 0.2) (layer "F.Cu") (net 11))
 (segment (start 144.778 111) (end 141.378 114.4) (width 0.2) (layer "F.Cu") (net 11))
 (segment (start 153.8 111) (end 144.778 111) (width 0.2) (layer "F.Cu") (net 11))
 (segment (start 152.4 112.268) (end 152.532 112.268) (width 0.2) (layer "F.Cu") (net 11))
 (segment (start 130.209861 114.4) (end 132.75 114.4) (width 0.2) (layer "F.Cu") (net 11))
 (segment (start 141.378 114.4) (end 132.75 114.4) (width 0.2) (layer "F.Cu") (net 11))
 (segment (start 153.8 104.5) (end 152.76 104.5) (width 0.2) (layer "F.Cu") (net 11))
 (segment (start 152.76 104.5) (end 152.4 104.14) (width 0.2) (layer "F.Cu") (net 11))
 (via (at 152.4 112.268) (size 0.46) (drill 0.2) (layers "F.Cu" "B.Cu") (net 11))
 (via (at 152.4 104.14) (size 0.46) (drill 0.2) (layers "F.Cu" "B.Cu") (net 11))
 (segment (start 152.146 112.268) (end 152.4 112.268) (width 0.2) (layer "B.Cu") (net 11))
 (segment (start 151.892 104.648) (end 151.892 112.014) (width 0.2) (layer "B.Cu") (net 11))
 (segment (start 152.4 104.14) (end 151.892 104.648) (width 0.2) (layer "B.Cu") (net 11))
 (segment (start 151.892 112.014) (end 152.146 112.268) (width 0.2) (layer "B.Cu") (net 11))
 (segment (start 147.04 106.4) (end 148.64 108) (width 0.2) (layer "F.Cu") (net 14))
 (segment (start 148.64 108) (end 153.8 108) (width 0.2) (layer "F.Cu") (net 14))
 (segment (start 139.709861 106.4) (end 142.25 106.4) (width 0.2) (layer "F.Cu") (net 14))
 (segment (start 142.25 106.4) (end 147.04 106.4) (width 0.2) (layer "F.Cu") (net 14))
 (segment (start 137.909861 106.4) (end 138.790139 106.4) (width 0.2) (layer "F.Cu") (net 7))
 (segment (start 131.190139 112.8) (end 130.309861 112.8) (width 0.2) (layer "F.Cu") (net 6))
 (segment (start 139.809861 104.8) (end 140.690139 104.8) (width 0.2) (layer "F.Cu") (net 20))
 (segment (start 133.090139 111.2) (end 132.209861 111.2) (width 0.2) (layer "F.Cu") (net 19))
 (segment (start 141.709861 103.2) (end 142.590139 103.2) (width 0.2) (layer "F.Cu") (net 24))
 (segment (start 134.990139 109.6) (end 134.109861 109.6) (width 0.2) (layer "F.Cu") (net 9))
 (segment (start 143.609861 101.6) (end 144.490139 101.6) (width 0.2) (layer "F.Cu") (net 1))
 (segment (start 127.390139 116) (end 126.509861 116) (width 0.2) (layer "F.Cu") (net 22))
 (segment (start 136.890139 108) (end 136.009861 108) (width 0.2) (layer "F.Cu") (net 4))
 (segment (start 145.509861 100) (end 146.390139 100) (width 0.2) (layer "F.Cu") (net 5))
 (segment (start 128.409861 114.4) (end 129.290139 114.4) (width 0.2) (layer "F.Cu") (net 23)))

